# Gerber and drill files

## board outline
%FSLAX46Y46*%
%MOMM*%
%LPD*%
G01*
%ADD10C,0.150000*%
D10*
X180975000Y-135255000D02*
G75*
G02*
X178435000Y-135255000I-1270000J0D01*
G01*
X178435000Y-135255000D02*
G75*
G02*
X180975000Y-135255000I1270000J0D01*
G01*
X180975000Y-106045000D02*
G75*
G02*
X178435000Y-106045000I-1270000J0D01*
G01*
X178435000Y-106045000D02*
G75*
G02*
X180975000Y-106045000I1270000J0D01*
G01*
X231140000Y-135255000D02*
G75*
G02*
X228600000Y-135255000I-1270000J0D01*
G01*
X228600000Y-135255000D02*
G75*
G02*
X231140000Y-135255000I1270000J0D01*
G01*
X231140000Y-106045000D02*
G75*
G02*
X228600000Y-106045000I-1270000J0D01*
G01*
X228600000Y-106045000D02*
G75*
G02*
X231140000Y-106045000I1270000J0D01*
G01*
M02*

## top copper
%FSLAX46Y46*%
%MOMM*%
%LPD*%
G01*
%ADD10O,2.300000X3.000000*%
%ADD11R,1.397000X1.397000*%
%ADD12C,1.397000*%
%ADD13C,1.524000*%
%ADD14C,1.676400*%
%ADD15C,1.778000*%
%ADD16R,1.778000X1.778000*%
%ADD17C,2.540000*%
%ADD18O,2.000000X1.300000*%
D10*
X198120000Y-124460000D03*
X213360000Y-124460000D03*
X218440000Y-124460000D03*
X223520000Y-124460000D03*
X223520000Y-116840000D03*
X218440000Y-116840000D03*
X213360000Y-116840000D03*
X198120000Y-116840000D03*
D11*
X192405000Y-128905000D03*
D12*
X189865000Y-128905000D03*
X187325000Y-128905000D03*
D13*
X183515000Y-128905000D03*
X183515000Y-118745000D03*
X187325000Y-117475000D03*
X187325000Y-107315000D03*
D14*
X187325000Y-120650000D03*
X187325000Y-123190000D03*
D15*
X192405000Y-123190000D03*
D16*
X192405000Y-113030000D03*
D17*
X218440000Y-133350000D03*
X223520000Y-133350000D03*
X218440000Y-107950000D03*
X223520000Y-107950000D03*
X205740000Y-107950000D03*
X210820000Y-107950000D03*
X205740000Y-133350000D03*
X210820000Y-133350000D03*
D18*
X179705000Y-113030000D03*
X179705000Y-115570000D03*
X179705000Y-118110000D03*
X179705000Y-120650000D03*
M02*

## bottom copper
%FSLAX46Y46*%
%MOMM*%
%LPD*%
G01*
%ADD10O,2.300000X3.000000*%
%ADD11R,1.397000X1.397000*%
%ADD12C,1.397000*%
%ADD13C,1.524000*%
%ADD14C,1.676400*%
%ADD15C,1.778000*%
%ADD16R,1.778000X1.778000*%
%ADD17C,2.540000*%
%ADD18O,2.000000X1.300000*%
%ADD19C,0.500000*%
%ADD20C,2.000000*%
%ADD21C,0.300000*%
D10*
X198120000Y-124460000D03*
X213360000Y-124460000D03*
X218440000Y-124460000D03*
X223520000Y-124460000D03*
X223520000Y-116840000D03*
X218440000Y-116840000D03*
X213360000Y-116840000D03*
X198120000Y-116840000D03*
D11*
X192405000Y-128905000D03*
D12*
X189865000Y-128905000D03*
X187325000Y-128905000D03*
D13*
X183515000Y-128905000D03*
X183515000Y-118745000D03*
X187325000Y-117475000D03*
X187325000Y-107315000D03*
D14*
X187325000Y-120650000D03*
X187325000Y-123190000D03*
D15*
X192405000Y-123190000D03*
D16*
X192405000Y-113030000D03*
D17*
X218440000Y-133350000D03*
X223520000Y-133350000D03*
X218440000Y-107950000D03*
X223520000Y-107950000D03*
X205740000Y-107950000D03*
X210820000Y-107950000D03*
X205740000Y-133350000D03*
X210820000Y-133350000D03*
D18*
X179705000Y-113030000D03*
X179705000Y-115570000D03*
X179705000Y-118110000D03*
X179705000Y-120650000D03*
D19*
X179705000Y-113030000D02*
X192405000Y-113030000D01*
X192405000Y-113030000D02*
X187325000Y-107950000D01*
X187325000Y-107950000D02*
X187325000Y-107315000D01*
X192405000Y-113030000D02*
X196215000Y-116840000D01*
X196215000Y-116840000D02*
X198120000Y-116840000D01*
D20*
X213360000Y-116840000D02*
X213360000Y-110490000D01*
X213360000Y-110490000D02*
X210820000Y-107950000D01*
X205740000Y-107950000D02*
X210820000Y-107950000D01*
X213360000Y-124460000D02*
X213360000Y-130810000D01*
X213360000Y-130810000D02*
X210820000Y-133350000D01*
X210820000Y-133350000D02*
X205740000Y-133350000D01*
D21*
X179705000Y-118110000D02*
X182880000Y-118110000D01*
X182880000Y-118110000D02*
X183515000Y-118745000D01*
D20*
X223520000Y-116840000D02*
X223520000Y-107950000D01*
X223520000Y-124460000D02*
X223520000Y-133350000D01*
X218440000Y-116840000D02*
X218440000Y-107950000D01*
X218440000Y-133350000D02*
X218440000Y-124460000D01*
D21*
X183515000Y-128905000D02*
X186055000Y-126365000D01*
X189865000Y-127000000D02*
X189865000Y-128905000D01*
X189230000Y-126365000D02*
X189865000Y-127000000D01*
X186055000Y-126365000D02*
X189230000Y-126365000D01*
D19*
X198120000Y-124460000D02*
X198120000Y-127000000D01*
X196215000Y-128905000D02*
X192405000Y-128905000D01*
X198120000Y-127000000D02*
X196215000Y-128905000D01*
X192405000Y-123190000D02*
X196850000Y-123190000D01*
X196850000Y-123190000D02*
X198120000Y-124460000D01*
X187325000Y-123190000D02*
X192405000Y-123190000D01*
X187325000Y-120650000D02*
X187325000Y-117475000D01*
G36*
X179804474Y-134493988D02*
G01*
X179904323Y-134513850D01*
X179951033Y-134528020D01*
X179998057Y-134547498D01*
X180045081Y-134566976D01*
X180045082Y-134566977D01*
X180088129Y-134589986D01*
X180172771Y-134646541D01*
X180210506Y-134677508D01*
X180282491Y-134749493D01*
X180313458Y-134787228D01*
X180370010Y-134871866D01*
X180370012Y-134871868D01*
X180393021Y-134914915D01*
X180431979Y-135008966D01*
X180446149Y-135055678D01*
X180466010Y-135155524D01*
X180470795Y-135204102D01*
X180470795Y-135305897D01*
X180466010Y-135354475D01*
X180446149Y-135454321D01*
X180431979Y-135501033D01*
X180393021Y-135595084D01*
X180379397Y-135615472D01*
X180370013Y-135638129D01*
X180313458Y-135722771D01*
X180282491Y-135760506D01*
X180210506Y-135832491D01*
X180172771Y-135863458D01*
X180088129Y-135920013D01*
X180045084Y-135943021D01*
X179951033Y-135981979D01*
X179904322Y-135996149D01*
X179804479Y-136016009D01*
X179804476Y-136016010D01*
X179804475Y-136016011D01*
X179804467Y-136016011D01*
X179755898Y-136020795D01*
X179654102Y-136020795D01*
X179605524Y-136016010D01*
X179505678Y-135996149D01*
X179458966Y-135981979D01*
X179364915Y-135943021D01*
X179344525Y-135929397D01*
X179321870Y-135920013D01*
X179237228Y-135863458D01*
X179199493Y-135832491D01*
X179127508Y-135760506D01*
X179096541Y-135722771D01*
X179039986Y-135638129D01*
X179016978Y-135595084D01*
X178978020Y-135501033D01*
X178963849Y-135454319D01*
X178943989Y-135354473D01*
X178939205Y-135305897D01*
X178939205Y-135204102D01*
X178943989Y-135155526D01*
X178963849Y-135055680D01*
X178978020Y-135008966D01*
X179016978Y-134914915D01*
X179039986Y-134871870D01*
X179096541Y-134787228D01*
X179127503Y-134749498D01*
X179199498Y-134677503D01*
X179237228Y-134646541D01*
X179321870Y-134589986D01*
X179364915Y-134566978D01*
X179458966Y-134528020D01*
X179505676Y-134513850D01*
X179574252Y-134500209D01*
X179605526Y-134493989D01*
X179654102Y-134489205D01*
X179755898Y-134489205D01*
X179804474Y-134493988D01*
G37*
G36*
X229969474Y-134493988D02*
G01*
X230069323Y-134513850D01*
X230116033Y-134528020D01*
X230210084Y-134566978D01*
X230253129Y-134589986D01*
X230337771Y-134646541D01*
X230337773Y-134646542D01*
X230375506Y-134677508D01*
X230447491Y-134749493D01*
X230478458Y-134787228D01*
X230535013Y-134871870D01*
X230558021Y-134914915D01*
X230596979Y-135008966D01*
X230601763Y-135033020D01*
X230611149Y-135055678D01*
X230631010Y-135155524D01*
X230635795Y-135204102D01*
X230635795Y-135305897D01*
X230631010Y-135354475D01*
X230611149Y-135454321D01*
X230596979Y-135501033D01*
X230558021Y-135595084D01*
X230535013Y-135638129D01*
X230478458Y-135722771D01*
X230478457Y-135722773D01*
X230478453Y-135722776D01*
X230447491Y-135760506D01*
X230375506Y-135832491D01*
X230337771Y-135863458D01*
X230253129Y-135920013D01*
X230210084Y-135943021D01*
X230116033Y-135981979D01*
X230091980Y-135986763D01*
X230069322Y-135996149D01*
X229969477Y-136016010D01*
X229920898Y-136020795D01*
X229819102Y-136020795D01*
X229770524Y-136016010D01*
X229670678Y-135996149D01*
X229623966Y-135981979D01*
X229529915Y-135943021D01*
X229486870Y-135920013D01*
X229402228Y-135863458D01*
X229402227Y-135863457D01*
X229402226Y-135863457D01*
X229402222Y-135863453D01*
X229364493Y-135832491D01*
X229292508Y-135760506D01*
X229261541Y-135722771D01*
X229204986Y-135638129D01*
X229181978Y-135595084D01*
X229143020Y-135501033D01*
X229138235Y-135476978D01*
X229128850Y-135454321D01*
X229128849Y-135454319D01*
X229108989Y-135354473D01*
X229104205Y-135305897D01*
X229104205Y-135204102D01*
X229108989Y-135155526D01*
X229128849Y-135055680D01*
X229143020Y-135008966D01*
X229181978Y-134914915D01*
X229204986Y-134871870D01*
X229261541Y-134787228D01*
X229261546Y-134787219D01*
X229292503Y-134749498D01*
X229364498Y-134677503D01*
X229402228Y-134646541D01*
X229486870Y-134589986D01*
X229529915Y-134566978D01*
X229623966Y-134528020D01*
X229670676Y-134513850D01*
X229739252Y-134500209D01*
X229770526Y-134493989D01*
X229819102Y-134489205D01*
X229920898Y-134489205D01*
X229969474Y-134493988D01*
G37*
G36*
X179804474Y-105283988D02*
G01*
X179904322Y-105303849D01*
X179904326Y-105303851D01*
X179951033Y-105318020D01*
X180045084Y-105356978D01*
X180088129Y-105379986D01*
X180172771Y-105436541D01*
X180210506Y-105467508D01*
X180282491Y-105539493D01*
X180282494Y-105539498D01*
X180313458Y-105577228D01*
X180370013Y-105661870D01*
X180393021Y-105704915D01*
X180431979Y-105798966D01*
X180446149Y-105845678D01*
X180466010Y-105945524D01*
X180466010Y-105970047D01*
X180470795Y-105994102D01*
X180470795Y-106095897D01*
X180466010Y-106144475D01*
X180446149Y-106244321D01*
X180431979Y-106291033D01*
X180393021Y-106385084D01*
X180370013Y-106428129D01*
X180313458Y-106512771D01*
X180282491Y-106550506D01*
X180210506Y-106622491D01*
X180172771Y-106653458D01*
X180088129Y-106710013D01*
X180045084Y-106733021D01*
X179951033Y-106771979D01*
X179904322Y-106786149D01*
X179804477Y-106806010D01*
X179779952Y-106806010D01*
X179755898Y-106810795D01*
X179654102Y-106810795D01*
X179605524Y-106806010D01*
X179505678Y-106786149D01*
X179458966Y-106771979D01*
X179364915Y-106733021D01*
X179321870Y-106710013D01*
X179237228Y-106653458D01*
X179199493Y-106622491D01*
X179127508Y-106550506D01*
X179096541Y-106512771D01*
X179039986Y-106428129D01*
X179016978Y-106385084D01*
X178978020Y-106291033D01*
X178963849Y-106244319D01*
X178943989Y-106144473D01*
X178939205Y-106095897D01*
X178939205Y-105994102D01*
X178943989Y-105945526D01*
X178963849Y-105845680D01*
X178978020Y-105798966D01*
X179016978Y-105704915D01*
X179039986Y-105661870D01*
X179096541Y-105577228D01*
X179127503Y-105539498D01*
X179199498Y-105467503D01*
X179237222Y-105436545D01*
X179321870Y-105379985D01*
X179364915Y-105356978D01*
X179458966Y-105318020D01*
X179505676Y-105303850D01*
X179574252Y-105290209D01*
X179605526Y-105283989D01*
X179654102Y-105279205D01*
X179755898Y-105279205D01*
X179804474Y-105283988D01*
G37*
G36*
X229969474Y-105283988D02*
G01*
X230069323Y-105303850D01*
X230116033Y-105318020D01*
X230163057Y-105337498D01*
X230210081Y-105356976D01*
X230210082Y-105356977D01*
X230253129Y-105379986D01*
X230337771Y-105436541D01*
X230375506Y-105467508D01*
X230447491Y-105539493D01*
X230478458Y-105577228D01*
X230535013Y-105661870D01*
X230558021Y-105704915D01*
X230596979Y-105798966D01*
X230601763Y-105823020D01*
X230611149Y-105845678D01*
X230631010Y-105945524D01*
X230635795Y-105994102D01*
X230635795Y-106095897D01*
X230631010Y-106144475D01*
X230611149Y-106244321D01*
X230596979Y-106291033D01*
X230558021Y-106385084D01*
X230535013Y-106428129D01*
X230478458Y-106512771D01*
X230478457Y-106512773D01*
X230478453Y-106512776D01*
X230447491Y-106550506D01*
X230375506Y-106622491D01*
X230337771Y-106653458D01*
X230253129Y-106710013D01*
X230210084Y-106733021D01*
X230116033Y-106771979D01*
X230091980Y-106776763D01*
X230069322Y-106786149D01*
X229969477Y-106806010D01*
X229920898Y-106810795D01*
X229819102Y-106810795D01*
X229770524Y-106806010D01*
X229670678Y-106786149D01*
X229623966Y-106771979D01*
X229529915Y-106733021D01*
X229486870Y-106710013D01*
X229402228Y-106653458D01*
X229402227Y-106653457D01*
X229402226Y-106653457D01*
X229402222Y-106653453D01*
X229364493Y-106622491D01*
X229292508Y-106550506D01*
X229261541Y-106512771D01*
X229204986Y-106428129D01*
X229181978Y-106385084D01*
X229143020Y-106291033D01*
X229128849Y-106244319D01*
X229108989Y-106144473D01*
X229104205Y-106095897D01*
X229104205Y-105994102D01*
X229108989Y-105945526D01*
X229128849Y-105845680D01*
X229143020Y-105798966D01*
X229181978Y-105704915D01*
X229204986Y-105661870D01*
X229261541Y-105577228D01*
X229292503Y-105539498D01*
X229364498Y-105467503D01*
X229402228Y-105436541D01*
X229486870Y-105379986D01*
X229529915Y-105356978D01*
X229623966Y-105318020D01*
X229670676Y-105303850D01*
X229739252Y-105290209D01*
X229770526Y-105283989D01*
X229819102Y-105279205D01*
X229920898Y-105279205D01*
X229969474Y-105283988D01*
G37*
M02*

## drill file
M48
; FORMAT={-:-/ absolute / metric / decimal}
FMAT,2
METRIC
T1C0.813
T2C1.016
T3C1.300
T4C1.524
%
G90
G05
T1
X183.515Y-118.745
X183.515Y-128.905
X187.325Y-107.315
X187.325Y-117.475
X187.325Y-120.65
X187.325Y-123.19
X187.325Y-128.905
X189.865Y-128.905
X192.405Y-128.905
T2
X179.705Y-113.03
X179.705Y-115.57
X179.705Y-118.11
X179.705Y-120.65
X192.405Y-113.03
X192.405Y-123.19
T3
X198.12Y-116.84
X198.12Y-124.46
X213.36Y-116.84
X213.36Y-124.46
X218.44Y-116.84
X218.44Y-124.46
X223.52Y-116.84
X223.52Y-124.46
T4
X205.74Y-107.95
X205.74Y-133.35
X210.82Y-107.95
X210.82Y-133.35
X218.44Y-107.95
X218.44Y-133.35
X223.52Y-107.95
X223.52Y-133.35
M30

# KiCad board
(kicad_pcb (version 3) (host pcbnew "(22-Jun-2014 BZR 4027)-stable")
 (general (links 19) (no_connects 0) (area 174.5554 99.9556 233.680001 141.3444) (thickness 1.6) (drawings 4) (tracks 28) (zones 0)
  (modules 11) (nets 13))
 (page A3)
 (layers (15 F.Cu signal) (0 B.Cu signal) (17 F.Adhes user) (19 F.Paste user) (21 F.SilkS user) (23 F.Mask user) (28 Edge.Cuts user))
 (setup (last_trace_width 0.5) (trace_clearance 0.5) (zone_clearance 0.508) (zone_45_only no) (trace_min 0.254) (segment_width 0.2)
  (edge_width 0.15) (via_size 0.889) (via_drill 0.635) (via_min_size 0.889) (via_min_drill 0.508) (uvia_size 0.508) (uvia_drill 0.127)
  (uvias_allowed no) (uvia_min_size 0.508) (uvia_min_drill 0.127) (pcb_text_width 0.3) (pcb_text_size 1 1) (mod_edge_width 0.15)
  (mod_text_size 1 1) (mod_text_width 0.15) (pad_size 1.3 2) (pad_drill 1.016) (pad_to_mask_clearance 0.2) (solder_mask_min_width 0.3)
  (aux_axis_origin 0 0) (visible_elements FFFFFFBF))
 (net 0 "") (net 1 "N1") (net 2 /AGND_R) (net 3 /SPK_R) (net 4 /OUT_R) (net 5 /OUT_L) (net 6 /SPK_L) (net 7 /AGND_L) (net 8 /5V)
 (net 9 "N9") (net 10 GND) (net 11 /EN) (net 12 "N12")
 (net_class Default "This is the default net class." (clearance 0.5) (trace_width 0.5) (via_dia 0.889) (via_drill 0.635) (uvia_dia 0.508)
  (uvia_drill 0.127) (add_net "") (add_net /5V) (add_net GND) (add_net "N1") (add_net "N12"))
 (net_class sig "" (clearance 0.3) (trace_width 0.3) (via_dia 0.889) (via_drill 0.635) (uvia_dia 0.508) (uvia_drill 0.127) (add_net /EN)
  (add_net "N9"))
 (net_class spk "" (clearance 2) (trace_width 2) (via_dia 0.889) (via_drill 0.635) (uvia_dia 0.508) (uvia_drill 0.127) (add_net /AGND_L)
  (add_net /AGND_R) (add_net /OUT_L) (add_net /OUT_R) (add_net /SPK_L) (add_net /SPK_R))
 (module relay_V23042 (layer F.Cu) (at 214.63 120.65)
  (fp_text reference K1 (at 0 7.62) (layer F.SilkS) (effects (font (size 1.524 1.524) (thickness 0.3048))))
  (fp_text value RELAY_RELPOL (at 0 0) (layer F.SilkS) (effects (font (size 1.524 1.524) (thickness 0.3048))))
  (pad 2 thru_hole oval (at -16.51 3.81) (size 2.3 3) (drill 1.3) (layers *.Cu *.Mask F.SilkS) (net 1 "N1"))
  (pad 3 thru_hole oval (at -1.27 3.81) (size 2.3 3) (drill 1.3) (layers *.Cu *.Mask F.SilkS) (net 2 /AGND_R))
  (pad 4 thru_hole oval (at 3.81 3.81) (size 2.3 3) (drill 1.3) (layers *.Cu *.Mask F.SilkS) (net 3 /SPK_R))
  (pad 5 thru_hole oval (at 8.89 3.81) (size 2.3 3) (drill 1.3) (layers *.Cu *.Mask F.SilkS) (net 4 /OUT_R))
  (pad 8 thru_hole oval (at 8.89 -3.81) (size 2.3 3) (drill 1.3) (layers *.Cu *.Mask F.SilkS) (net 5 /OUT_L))
  (pad 7 thru_hole oval (at 3.81 -3.81) (size 2.3 3) (drill 1.3) (layers *.Cu *.Mask F.SilkS) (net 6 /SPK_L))
  (pad 6 thru_hole oval (at -1.27 -3.81) (size 2.3 3) (drill 1.3) (layers *.Cu *.Mask F.SilkS) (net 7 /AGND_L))
  (pad 1 thru_hole oval (at -16.51 -3.81) (size 2.3 3) (drill 1.3) (layers *.Cu *.Mask F.SilkS) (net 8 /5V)))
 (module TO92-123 (layer F.Cu) (at 191.135 130.175)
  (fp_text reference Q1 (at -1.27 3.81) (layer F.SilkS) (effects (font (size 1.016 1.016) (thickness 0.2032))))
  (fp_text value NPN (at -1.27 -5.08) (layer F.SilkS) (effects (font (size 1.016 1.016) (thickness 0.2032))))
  (pad 3 thru_hole rect (at 1.27 -1.27) (size 1.397 1.397) (drill 0.8128) (layers *.Cu *.Mask F.SilkS) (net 1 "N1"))
  (pad 2 thru_hole circle (at -1.27 -1.27) (size 1.397 1.397) (drill 0.8128) (layers *.Cu *.Mask F.SilkS) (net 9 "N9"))
  (pad 1 thru_hole circle (at -3.81 -1.27) (size 1.397 1.397) (drill 0.8128) (layers *.Cu *.Mask F.SilkS) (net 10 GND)))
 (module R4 (layer F.Cu) (at 183.515 123.825 90) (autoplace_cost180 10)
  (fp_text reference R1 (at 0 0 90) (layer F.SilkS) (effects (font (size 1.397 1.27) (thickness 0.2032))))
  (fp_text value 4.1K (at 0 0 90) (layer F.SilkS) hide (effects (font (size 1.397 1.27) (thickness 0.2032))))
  (pad 1 thru_hole circle (at -5.08 0 90) (size 1.524 1.524) (drill 0.8128) (layers *.Cu *.Mask F.SilkS) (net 9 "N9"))
  (pad 2 thru_hole circle (at 5.08 0 90) (size 1.524 1.524) (drill 0.8128) (layers *.Cu *.Mask F.SilkS) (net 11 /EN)))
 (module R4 (layer F.Cu) (at 187.325 112.395 90) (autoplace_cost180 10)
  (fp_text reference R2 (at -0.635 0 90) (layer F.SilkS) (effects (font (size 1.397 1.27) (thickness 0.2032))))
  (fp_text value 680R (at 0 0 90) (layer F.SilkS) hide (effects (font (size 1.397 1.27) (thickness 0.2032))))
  (pad 1 thru_hole circle (at -5.08 0 90) (size 1.524 1.524) (drill 0.8128) (layers *.Cu *.Mask F.SilkS) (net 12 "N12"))
  (pad 2 thru_hole circle (at 5.08 0 90) (size 1.524 1.524) (drill 0.8128) (layers *.Cu *.Mask F.SilkS) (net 8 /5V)))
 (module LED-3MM (layer F.Cu) (at 187.325 121.92 270)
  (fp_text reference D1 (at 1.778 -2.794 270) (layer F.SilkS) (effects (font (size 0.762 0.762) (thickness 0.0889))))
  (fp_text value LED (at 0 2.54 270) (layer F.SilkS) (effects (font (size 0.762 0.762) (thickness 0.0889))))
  (pad 1 thru_hole circle (at -1.27 0 270) (size 1.6764 1.6764) (drill 0.8128) (layers *.Cu *.Mask F.SilkS) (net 12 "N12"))
  (pad 2 thru_hole circle (at 1.27 0 270) (size 1.6764 1.6764) (drill 0.8128) (layers *.Cu *.Mask F.SilkS) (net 1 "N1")))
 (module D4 (layer F.Cu) (at 192.405 118.11 90)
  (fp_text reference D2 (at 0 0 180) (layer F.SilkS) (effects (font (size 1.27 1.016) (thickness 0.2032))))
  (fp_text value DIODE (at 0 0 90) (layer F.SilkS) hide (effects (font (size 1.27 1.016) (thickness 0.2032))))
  (pad 1 thru_hole circle (at -5.08 0 90) (size 1.778 1.778) (drill 1.016) (layers *.Cu *.Mask F.SilkS) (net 1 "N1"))
  (pad 2 thru_hole rect (at 5.08 0 90) (size 1.778 1.778) (drill 1.016) (layers *.Cu *.Mask F.SilkS) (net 8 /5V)))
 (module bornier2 (layer F.Cu) (at 220.98 133.35)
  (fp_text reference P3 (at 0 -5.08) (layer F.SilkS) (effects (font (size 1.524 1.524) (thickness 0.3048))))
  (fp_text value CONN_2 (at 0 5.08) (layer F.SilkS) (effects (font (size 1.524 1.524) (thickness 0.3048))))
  (pad 1 thru_hole circle (at -2.54 0) (size 2.54 2.54) (drill 1.524) (layers *.Cu *.Mask F.SilkS) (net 3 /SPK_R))
  (pad 2 thru_hole circle (at 2.54 0) (size 2.54 2.54) (drill 1.524) (layers *.Cu *.Mask F.SilkS) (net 4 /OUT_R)))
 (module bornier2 (layer F.Cu) (at 220.98 107.95)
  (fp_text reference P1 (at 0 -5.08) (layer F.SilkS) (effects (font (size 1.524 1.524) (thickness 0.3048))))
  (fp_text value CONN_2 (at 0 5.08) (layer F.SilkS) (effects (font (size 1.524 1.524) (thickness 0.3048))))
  (pad 1 thru_hole circle (at -2.54 0) (size 2.54 2.54) (drill 1.524) (layers *.Cu *.Mask F.SilkS) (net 6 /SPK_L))
  (pad 2 thru_hole circle (at 2.54 0) (size 2.54 2.54) (drill 1.524) (layers *.Cu *.Mask F.SilkS) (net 5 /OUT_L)))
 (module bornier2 (layer F.Cu) (at 208.28 107.95)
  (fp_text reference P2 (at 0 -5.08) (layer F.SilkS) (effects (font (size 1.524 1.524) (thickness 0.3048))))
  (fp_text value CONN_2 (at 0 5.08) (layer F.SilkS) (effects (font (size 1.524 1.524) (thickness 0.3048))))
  (pad 1 thru_hole circle (at -2.54 0) (size 2.54 2.54) (drill 1.524) (layers *.Cu *.Mask F.SilkS) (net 7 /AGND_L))
  (pad 2 thru_hole circle (at 2.54 0) (size 2.54 2.54) (drill 1.524) (layers *.Cu *.Mask F.SilkS) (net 7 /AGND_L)))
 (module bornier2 (layer F.Cu) (at 208.28 133.35)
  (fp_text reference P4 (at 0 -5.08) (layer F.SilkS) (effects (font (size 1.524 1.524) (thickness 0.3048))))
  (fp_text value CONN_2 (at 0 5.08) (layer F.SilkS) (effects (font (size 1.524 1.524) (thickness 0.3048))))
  (pad 1 thru_hole circle (at -2.54 0) (size 2.54 2.54) (drill 1.524) (layers *.Cu *.Mask F.SilkS) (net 2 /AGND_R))
  (pad 2 thru_hole circle (at 2.54 0) (size 2.54 2.54) (drill 1.524) (layers *.Cu *.Mask F.SilkS) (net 2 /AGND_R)))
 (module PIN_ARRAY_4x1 (layer F.Cu) (at 179.705 116.84 270)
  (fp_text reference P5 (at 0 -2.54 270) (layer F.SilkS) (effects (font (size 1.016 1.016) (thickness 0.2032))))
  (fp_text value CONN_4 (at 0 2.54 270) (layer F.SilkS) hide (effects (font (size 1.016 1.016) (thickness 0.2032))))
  (pad 1 thru_hole oval (at -3.81 0 270) (size 1.3 2) (drill 1.016) (layers *.Cu *.Mask F.SilkS) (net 8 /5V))
  (pad 2 thru_hole oval (at -1.27 0 270) (size 1.3 2) (drill 1.016) (layers *.Cu *.Mask F.SilkS) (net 10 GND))
  (pad 3 thru_hole oval (at 1.27 0 270) (size 1.3 2) (drill 1.016) (layers *.Cu *.Mask F.SilkS) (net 11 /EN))
  (pad 4 thru_hole oval (at 3.81 0 270) (size 1.3 2) (drill 1.016) (layers *.Cu *.Mask F.SilkS) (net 10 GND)))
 (gr_circle (center 179.705 135.255) (end 180.975 135.255) (layer Edge.Cuts) (width 0.15))
 (gr_circle (center 179.705 106.045) (end 180.975 106.045) (layer Edge.Cuts) (width 0.15))
 (gr_circle (center 229.87 135.255) (end 231.14 135.255) (layer Edge.Cuts) (width 0.15))
 (gr_circle (center 229.87 106.045) (end 231.14 106.045) (layer Edge.Cuts) (width 0.15))
 (segment (start 179.705 113.03) (end 192.405 113.03) (width 0.5) (layer B.Cu) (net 8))
 (segment (start 192.405 113.03) (end 187.325 107.95) (width 0.5) (layer B.Cu) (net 8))
 (segment (start 187.325 107.95) (end 187.325 107.315) (width 0.5) (layer B.Cu) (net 8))
 (segment (start 192.405 113.03) (end 196.215 116.84) (width 0.5) (layer B.Cu) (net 8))
 (segment (start 196.215 116.84) (end 198.12 116.84) (width 0.5) (layer B.Cu) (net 8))
 (segment (start 213.36 116.84) (end 213.36 110.49) (width 2) (layer B.Cu) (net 7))
 (segment (start 213.36 110.49) (end 210.82 107.95) (width 2) (layer B.Cu) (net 7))
 (segment (start 205.74 107.95) (end 210.82 107.95) (width 2) (layer B.Cu) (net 7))
 (segment (start 213.36 124.46) (end 213.36 130.81) (width 2) (layer B.Cu) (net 2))
 (segment (start 213.36 130.81) (end 210.82 133.35) (width 2) (layer B.Cu) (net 2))
 (segment (start 210.82 133.35) (end 205.74 133.35) (width 2) (layer B.Cu) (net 2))
 (segment (start 179.705 118.11) (end 182.88 118.11) (width 0.3) (layer B.Cu) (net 11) (status 400000))
 (segment (start 182.88 118.11) (end 183.515 118.745) (width 0.3) (layer B.Cu) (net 11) (status 800000))
 (segment (start 223.52 116.84) (end 223.52 107.95) (width 2) (layer B.Cu) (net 5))
 (segment (start 223.52 124.46) (end 223.52 133.35) (width 2) (layer B.Cu) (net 4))
 (segment (start 218.44 116.84) (end 218.44 107.95) (width 2) (layer B.Cu) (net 6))
 (segment (start 218.44 133.35) (end 218.44 124.46) (width 2) (layer B.Cu) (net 3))
 (segment (start 183.515 128.905) (end 186.055 126.365) (width 0.3) (layer B.Cu) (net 9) (status 400000))
 (segment (start 189.865 127) (end 189.865 128.905) (width 0.3) (layer B.Cu) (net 9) (status 800000))
 (segment (start 189.23 126.365) (end 189.865 127) (width 0.3) (layer B.Cu) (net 9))
 (segment (start 186.055 126.365) (end 189.23 126.365) (width 0.3) (layer B.Cu) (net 9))
 (segment (start 198.12 124.46) (end 198.12 127) (width 0.5) (layer B.Cu) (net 1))
 (segment (start 196.215 128.905) (end 192.405 128.905) (width 0.5) (layer B.Cu) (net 1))
 (segment (start 198.12 127) (end 196.215 128.905) (width 0.5) (layer B.Cu) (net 1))
 (segment (start 192.405 123.19) (end 196.85 123.19) (width 0.5) (layer B.Cu) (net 1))
 (segment (start 196.85 123.19) (end 198.12 124.46) (width 0.5) (layer B.Cu) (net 1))
 (segment (start 187.325 123.19) (end 192.405 123.19) (width 0.5) (layer B.Cu) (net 1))
 (segment (start 187.325 120.65) (end 187.325 117.475) (width 0.5) (layer B.Cu) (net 12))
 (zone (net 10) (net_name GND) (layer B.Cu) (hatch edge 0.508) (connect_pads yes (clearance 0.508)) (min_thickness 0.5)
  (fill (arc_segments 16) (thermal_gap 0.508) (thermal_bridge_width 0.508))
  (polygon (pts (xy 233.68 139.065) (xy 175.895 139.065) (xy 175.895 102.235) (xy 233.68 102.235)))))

